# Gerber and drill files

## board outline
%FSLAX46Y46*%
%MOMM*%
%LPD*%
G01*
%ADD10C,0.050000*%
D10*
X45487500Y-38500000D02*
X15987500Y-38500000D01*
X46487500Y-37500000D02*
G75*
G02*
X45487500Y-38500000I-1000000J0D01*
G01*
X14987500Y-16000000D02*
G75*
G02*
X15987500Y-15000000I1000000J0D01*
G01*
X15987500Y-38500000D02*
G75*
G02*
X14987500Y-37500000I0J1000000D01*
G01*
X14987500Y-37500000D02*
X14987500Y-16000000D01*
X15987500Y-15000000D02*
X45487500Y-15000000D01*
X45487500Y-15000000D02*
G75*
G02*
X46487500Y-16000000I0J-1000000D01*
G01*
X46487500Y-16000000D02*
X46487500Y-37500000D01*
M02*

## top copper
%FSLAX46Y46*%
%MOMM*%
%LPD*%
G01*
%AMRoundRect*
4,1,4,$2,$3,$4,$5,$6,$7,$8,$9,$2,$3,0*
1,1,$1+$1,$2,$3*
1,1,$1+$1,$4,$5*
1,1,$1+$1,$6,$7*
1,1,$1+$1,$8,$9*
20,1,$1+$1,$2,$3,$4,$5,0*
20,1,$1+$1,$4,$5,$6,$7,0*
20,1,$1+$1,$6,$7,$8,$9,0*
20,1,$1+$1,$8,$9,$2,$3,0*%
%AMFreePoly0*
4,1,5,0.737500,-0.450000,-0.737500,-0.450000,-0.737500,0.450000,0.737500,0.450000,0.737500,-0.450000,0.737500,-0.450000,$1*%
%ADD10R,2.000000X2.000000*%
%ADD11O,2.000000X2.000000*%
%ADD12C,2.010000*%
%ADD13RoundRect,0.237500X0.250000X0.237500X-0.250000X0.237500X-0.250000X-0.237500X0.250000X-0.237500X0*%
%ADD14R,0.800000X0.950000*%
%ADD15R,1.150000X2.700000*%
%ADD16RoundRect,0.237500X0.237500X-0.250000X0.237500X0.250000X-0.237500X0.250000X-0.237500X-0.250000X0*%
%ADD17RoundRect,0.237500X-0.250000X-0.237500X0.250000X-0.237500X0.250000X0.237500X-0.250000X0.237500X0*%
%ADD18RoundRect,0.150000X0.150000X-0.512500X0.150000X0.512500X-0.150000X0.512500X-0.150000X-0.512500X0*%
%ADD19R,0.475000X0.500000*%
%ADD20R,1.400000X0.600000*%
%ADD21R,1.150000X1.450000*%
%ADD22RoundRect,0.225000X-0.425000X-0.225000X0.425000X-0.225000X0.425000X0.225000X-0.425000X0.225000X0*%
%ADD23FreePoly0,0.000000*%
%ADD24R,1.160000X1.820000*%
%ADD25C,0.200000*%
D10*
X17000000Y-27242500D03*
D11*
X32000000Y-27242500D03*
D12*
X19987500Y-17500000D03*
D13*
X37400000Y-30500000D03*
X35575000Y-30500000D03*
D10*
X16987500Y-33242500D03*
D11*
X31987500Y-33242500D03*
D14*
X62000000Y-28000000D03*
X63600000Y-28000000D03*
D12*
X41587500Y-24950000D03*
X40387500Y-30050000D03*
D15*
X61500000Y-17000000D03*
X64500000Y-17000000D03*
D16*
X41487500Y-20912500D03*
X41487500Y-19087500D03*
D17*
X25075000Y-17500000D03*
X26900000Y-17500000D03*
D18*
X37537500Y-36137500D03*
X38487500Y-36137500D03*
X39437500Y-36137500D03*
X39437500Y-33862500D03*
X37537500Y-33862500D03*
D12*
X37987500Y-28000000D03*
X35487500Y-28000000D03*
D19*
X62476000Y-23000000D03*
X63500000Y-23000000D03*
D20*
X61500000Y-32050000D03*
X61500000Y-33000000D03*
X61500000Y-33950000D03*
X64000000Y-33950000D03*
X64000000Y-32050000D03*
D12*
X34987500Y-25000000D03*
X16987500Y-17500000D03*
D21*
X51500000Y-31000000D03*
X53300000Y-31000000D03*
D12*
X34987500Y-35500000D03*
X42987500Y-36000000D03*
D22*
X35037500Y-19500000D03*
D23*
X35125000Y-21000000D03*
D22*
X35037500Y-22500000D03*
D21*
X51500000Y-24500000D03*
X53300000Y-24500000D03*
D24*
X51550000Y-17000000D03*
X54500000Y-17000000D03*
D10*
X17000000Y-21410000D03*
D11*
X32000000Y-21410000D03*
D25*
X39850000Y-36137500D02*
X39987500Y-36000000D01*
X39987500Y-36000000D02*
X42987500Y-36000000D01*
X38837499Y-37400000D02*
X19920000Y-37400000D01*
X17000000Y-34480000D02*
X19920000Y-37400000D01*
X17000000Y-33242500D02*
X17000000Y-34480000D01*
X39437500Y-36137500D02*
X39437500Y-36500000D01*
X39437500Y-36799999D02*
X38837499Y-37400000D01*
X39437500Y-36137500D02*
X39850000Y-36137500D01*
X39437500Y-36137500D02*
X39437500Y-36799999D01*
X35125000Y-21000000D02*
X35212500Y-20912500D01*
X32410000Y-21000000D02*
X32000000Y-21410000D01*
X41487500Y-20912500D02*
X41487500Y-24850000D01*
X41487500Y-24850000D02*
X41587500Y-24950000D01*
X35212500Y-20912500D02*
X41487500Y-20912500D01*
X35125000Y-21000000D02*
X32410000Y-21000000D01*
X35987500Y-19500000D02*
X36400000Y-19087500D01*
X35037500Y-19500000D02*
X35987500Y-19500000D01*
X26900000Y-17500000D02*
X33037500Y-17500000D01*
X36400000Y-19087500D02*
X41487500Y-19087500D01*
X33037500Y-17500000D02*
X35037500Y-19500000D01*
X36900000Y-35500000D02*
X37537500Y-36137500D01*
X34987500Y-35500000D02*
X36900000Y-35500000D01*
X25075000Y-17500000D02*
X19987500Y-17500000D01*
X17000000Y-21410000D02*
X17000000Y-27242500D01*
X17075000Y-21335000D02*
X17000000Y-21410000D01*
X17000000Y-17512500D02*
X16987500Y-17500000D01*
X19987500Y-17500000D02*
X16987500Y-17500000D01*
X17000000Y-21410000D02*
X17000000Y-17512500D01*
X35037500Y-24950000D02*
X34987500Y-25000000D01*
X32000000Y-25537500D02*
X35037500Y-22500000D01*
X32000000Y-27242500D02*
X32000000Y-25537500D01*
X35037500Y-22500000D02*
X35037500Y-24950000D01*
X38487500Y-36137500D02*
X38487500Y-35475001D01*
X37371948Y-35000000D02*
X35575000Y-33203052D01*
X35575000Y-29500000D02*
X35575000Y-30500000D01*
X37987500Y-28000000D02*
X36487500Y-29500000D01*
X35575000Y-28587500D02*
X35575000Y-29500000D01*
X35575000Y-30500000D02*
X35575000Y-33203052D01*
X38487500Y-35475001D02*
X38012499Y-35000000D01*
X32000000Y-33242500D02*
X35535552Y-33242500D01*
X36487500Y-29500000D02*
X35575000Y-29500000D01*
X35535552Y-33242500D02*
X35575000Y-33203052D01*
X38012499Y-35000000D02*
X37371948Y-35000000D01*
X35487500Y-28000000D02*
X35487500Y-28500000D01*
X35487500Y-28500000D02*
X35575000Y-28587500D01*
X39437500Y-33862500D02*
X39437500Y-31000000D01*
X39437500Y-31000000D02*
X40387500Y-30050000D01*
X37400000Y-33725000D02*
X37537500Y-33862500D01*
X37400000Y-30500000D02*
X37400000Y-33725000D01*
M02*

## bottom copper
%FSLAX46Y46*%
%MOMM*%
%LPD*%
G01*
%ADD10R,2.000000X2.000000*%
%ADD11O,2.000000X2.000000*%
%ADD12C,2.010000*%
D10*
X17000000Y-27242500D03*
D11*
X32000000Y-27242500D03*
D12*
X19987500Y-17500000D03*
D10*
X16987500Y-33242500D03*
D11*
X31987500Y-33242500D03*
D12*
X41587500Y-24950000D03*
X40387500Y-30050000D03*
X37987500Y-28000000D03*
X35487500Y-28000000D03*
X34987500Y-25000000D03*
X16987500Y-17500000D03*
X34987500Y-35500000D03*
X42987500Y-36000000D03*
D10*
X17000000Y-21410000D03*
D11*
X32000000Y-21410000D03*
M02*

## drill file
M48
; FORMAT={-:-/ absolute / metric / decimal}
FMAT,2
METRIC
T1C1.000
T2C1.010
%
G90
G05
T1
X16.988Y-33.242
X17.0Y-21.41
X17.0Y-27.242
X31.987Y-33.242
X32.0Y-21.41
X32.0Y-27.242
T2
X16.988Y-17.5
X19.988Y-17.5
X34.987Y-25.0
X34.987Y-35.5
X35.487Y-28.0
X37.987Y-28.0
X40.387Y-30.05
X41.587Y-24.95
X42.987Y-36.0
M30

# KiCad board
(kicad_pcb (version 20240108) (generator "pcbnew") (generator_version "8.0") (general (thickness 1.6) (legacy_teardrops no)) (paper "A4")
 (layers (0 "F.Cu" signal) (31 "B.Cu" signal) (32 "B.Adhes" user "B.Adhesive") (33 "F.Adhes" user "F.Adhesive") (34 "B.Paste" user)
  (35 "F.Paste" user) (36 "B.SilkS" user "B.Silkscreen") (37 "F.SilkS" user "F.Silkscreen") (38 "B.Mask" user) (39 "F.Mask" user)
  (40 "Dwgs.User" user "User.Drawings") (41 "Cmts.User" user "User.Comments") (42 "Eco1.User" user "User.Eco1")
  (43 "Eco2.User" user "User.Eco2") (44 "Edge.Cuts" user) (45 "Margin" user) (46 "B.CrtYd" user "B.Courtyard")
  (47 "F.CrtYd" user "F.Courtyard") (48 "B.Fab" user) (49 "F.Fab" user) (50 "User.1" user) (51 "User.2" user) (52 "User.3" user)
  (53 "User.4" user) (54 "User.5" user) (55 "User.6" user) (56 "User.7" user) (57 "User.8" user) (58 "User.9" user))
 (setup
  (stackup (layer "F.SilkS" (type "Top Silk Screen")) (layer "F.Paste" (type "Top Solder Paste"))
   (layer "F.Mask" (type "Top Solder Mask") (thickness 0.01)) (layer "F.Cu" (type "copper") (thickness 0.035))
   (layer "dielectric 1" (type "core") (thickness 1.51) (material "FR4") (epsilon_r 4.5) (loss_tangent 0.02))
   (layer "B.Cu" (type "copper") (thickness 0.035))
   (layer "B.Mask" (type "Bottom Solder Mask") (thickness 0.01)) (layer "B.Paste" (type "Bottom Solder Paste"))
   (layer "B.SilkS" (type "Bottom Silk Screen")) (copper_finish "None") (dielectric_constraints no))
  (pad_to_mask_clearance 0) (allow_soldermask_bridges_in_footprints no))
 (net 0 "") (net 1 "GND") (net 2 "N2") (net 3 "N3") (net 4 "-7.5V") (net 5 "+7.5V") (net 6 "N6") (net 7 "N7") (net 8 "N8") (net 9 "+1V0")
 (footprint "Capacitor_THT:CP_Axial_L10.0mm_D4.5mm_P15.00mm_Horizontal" (layer "F.Cu") (at 17 27.2425)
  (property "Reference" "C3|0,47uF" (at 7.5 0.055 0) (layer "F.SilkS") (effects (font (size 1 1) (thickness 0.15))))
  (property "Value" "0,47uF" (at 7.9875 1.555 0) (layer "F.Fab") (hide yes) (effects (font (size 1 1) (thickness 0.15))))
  (pad "2" thru_hole rect (at 0 0) (size 2 2) (drill 1) (layers "*.Cu" "*.Mask") (remove_unused_layers no) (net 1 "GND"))
  (pad "2" thru_hole oval (at 15 0) (size 2 2) (drill 1) (layers "*.Cu" "*.Mask") (remove_unused_layers no) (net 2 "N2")))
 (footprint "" (layer "F.Cu") (at 19.9875 17.5)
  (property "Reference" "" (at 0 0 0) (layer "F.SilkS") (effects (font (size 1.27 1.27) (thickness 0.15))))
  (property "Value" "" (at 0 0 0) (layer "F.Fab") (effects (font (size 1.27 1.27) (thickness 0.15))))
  (pad "4" thru_hole circle (at 0 0 270) (size 2.01 2.01) (drill 1.01) (layers "*.Cu" "*.Mask") (remove_unused_layers no) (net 1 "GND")))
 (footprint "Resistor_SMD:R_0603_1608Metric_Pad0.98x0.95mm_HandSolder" (layer "F.Cu") (at 36.4875 30.5 180)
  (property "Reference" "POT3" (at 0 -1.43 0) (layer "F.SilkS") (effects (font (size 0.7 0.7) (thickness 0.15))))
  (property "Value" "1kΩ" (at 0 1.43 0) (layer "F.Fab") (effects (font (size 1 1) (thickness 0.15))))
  (pad "1" smd roundrect (at -0.9125 0 180) (size 0.975 0.95) (layers "F.Cu" "F.Paste" "F.Mask") (roundrect_rratio 0.25) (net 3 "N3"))
  (pad "2" smd roundrect (at 0.9125 0 180) (size 0.975 0.95) (layers "F.Cu" "F.Paste" "F.Mask") (roundrect_rratio 0.25) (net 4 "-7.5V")))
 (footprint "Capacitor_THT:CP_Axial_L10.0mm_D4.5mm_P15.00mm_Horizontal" (layer "F.Cu") (at 16.9875 33.2425)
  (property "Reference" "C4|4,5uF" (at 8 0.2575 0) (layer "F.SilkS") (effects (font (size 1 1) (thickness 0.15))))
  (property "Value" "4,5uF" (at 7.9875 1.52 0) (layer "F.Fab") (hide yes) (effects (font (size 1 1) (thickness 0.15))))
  (pad "1" thru_hole rect (at 0 0) (size 2 2) (drill 1) (layers "*.Cu" "*.Mask") (remove_unused_layers no) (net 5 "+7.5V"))
  (pad "2" thru_hole oval (at 15 0) (size 2 2) (drill 1) (layers "*.Cu" "*.Mask") (remove_unused_layers no) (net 4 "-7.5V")))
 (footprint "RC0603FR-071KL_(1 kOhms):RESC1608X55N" (layer "F.Cu") (at 62.8 28)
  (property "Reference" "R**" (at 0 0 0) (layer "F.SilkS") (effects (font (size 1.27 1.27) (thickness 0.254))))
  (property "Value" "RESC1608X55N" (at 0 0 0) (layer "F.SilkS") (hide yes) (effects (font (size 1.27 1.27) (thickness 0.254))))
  (pad "1" smd rect (at -0.8 0) (size 0.8 0.95) (layers "F.Cu" "F.Paste" "F.Mask"))
  (pad "2" smd rect (at 0.8 0) (size 0.8 0.95) (layers "F.Cu" "F.Paste" "F.Mask")))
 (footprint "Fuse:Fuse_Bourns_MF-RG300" (layer "F.Cu") (at 41.5875 24.95 -90)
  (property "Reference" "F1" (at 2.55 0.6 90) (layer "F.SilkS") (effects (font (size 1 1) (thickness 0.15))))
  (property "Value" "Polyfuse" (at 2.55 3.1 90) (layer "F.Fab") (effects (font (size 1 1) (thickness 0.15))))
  (pad "1" thru_hole circle (at 0 0 270) (size 2.01 2.01) (drill 1.01) (layers "*.Cu" "*.Mask") (remove_unused_layers no) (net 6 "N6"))
  (pad "2" thru_hole circle (at 5.1 1.2 270) (size 2.01 2.01) (drill 1.01) (layers "*.Cu" "*.Mask") (remove_unused_layers no) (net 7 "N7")))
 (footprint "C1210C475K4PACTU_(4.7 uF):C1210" (layer "F.Cu") (at 63 17)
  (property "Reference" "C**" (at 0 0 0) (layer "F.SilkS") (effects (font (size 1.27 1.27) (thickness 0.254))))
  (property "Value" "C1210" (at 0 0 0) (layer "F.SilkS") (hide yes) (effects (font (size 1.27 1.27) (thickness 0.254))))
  (pad "1" smd rect (at -1.5 0) (size 1.15 2.7) (layers "F.Cu" "F.Paste" "F.Mask"))
  (pad "2" smd rect (at 1.5 0) (size 1.15 2.7) (layers "F.Cu" "F.Paste" "F.Mask")))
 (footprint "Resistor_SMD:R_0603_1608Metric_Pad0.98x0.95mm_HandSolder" (layer "F.Cu") (at 41.4875 20 90)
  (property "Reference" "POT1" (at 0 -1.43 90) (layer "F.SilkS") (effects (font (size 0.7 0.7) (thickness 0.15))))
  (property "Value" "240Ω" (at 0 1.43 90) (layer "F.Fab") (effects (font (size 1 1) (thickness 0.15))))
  (pad "1" smd roundrect (at -0.9125 0 90) (size 0.975 0.95) (layers "F.Cu" "F.Paste" "F.Mask") (roundrect_rratio 0.25) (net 6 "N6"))
  (pad "2" smd roundrect (at 0.9125 0 90) (size 0.975 0.95) (layers "F.Cu" "F.Paste" "F.Mask") (roundrect_rratio 0.25) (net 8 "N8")))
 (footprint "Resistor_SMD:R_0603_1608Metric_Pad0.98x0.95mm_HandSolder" (layer "F.Cu") (at 25.9875 17.5)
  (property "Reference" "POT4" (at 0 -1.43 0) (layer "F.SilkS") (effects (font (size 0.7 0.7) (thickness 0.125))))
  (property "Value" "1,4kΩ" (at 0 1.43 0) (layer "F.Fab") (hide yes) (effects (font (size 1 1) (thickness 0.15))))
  (pad "1" smd roundrect (at -0.9125 0) (size 0.975 0.95) (layers "F.Cu" "F.Paste" "F.Mask") (roundrect_rratio 0.25) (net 1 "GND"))
  (pad "2" smd roundrect (at 0.9125 0) (size 0.975 0.95) (layers "F.Cu" "F.Paste" "F.Mask") (roundrect_rratio 0.25) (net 8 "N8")))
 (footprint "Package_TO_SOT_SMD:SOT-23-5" (layer "F.Cu") (at 38.4875 35 90)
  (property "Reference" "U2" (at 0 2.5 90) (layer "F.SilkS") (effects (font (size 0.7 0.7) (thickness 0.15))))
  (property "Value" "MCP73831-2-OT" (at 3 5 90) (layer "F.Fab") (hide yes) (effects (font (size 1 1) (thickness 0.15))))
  (pad "1" smd roundrect (at -1.1375 -0.95 90) (size 1.325 0.6) (layers "F.Cu" "F.Paste" "F.Mask") (roundrect_rratio 0.25) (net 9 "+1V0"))
  (pad "2" smd roundrect (at -1.1375 0 90) (size 1.325 0.6) (layers "F.Cu" "F.Paste" "F.Mask") (roundrect_rratio 0.25) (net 4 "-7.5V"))
  (pad "3" smd roundrect (at -1.1375 0.95 90) (size 1.325 0.6) (layers "F.Cu" "F.Paste" "F.Mask") (roundrect_rratio 0.25) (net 5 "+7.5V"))
  (pad "4" smd roundrect (at 1.1375 0.95 90) (size 1.325 0.6) (layers "F.Cu" "F.Paste" "F.Mask") (roundrect_rratio 0.25) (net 7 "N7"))
  (pad "5" smd roundrect (at 1.1375 -0.95 90) (size 1.325 0.6) (layers "F.Cu" "F.Paste" "F.Mask") (roundrect_rratio 0.25) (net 3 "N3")))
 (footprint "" (layer "F.Cu") (at 37.9875 28)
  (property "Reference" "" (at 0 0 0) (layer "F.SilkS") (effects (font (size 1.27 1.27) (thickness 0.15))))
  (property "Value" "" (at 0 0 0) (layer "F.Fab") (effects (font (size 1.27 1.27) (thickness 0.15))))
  (pad "1" thru_hole circle (at 0 0 270) (size 2.01 2.01) (drill 1.01) (layers "*.Cu" "*.Mask") (remove_unused_layers no) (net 4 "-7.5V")))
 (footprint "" (layer "F.Cu") (at 35.4875 28)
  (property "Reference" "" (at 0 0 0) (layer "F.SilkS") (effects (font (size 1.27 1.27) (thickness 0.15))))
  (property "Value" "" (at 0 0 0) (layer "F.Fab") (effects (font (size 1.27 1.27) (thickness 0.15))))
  (pad "1" thru_hole circle (at 0 0 270) (size 2.01 2.01) (drill 1.01) (layers "*.Cu" "*.Mask") (remove_unused_layers no) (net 4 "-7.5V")))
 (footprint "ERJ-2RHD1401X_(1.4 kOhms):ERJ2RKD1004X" (layer "F.Cu") (at 62.988 23)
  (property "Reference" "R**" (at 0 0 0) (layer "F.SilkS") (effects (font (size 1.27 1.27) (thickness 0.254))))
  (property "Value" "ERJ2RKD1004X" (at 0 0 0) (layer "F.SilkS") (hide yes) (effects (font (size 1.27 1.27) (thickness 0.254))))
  (pad "1" smd rect (at -0.512 0) (size 0.475 0.5) (layers "F.Cu" "F.Paste" "F.Mask"))
  (pad "2" smd rect (at 0.512 0) (size 0.475 0.5) (layers "F.Cu" "F.Paste" "F.Mask")))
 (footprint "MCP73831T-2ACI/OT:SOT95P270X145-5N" (layer "F.Cu") (at 62.75 33)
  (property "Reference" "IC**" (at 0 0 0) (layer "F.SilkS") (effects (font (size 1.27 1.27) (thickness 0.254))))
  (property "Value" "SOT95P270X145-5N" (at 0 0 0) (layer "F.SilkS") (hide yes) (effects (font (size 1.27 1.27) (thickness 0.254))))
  (pad "1" smd rect (at -1.25 -0.95 90) (size 0.6 1.4) (layers "F.Cu" "F.Paste" "F.Mask"))
  (pad "2" smd rect (at -1.25 0 90) (size 0.6 1.4) (layers "F.Cu" "F.Paste" "F.Mask"))
  (pad "3" smd rect (at -1.25 0.95 90) (size 0.6 1.4) (layers "F.Cu" "F.Paste" "F.Mask"))
  (pad "4" smd rect (at 1.25 0.95 90) (size 0.6 1.4) (layers "F.Cu" "F.Paste" "F.Mask"))
  (pad "5" smd rect (at 1.25 -0.95 90) (size 0.6 1.4) (layers "F.Cu" "F.Paste" "F.Mask")))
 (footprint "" (layer "F.Cu") (at 34.9875 25)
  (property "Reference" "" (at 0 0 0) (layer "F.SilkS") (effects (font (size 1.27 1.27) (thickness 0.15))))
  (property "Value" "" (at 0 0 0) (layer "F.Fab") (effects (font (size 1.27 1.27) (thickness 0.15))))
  (pad "1" thru_hole circle (at 0 0 270) (size 2.01 2.01) (drill 1.01) (layers "*.Cu" "*.Mask") (remove_unused_layers no) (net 2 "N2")))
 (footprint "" (layer "F.Cu") (at 16.9875 17.5)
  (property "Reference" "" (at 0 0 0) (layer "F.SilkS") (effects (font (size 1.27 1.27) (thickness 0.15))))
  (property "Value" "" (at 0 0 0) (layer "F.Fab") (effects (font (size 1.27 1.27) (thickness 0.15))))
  (pad "3" thru_hole circle (at 0 0 270) (size 2.01 2.01) (drill 1.01) (layers "*.Cu" "*.Mask") (remove_unused_layers no) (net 1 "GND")))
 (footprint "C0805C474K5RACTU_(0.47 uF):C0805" (layer "F.Cu") (at 52.4 31)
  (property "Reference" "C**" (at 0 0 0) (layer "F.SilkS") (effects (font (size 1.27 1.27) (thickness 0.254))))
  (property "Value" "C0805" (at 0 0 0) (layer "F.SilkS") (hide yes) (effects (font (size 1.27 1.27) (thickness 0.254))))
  (pad "1" smd rect (at -0.9 0) (size 1.15 1.45) (layers "F.Cu" "F.Paste" "F.Mask"))
  (pad "2" smd rect (at 0.9 0) (size 1.15 1.45) (layers "F.Cu" "F.Paste" "F.Mask")))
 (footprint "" (layer "F.Cu") (at 34.9875 35.5)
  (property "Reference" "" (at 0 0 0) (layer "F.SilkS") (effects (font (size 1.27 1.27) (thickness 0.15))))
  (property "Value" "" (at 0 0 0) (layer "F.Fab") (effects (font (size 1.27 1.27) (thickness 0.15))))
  (pad "1" thru_hole circle (at 0 0 270) (size 2.01 2.01) (drill 1.01) (layers "*.Cu" "*.Mask") (remove_unused_layers no) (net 9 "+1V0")))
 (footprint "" (layer "F.Cu") (at 42.9875 36)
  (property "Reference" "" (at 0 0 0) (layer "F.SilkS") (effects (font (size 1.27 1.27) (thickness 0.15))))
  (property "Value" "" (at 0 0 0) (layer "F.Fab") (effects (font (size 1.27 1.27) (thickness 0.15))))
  (pad "2" thru_hole circle (at 0 0 270) (size 2.01 2.01) (drill 1.01) (layers "*.Cu" "*.Mask") (remove_unused_layers no) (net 5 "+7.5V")))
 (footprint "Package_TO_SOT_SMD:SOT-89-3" (layer "F.Cu") (at 36.9875 21)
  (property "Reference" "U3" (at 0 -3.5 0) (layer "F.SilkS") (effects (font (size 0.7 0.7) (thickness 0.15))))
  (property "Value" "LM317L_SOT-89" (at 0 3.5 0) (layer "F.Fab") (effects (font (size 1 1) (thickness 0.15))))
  (pad "1" smd roundrect (at -1.95 -1.5) (size 1.3 0.9) (layers "F.Cu" "F.Paste" "F.Mask") (roundrect_rratio 0.25) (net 8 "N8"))
  (pad "2" smd custom (at -1.8625 0) (size 1.475 0.9) (layers "F.Cu" "F.Paste" "F.Mask") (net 6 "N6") (zone_connect 2)
   (thermal_bridge_angle 45) (options (clearance outline) (anchor rect)) (primitives))
  (pad "3" smd roundrect (at -1.95 1.5) (size 1.3 0.9) (layers "F.Cu" "F.Paste" "F.Mask") (roundrect_rratio 0.25) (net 2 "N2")))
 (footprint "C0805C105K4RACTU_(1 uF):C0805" (layer "F.Cu") (at 52.4 24.5)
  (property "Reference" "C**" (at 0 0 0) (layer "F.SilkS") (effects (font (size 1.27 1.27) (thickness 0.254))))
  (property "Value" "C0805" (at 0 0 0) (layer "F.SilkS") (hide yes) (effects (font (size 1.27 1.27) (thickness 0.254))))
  (pad "1" smd rect (at -0.9 0) (size 1.15 1.45) (layers "F.Cu" "F.Paste" "F.Mask"))
  (pad "2" smd rect (at 0.9 0) (size 1.15 1.45) (layers "F.Cu" "F.Paste" "F.Mask")))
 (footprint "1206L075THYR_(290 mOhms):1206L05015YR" (layer "F.Cu") (at 53.025 17)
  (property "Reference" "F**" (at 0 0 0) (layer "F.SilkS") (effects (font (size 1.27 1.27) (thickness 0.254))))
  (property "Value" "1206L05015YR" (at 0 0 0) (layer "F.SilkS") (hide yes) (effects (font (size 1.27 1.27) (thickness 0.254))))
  (pad "1" smd rect (at -1.475 0) (size 1.16 1.82) (layers "F.Cu" "F.Paste" "F.Mask"))
  (pad "2" smd rect (at 1.475 0) (size 1.16 1.82) (layers "F.Cu" "F.Paste" "F.Mask")))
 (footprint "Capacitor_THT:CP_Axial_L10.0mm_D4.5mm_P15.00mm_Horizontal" (layer "F.Cu") (at 17 21.41)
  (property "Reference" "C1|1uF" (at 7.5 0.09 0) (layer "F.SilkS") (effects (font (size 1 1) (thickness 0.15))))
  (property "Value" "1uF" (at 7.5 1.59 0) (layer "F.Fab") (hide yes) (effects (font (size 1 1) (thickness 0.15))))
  (pad "1" thru_hole rect (at 0 0) (size 2 2) (drill 1) (layers "*.Cu" "*.Mask") (remove_unused_layers no) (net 1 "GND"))
  (pad "2" thru_hole oval (at 15 0) (size 2 2) (drill 1) (layers "*.Cu" "*.Mask") (remove_unused_layers no) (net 6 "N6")))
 (gr_line (start 45.4875 38.5) (end 15.9875 38.5) (stroke (width 0.05) (type default)) (layer "Edge.Cuts"))
 (gr_arc (start 46.4875 37.5) (mid 46.194607 38.207107) (end 45.4875 38.5) (stroke (width 0.05) (type default)) (layer "Edge.Cuts"))
 (gr_arc (start 14.9875 16) (mid 15.280393 15.292893) (end 15.9875 15) (stroke (width 0.05) (type default)) (layer "Edge.Cuts"))
 (gr_arc (start 15.9875 38.5) (mid 15.280393 38.207107) (end 14.9875 37.5) (stroke (width 0.05) (type default)) (layer "Edge.Cuts"))
 (gr_line (start 14.9875 37.5) (end 14.9875 16) (stroke (width 0.05) (type default)) (layer "Edge.Cuts"))
 (gr_line (start 15.9875 15) (end 45.4875 15) (stroke (width 0.05) (type default)) (layer "Edge.Cuts"))
 (gr_arc (start 45.4875 15) (mid 46.194607 15.292893) (end 46.4875 16) (stroke (width 0.05) (type default)) (layer "Edge.Cuts"))
 (gr_line (start 46.4875 16) (end 46.4875 37.5) (stroke (width 0.05) (type default)) (layer "Edge.Cuts"))
 (segment (start 39.85 36.1375) (end 39.9875 36) (width 0.2) (layer "F.Cu") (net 5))
 (segment (start 39.9875 36) (end 42.9875 36) (width 0.2) (layer "F.Cu") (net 5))
 (segment (start 38.837499 37.4) (end 19.92 37.4) (width 0.2) (layer "F.Cu") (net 5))
 (segment (start 17 34.48) (end 19.92 37.4) (width 0.2) (layer "F.Cu") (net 5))
 (segment (start 17 33.2425) (end 17 34.48) (width 0.2) (layer "F.Cu") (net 5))
 (segment (start 39.4375 36.1375) (end 39.4375 36.5) (width 0.2) (layer "F.Cu") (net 5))
 (segment (start 39.4375 36.799999) (end 38.837499 37.4) (width 0.2) (layer "F.Cu") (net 5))
 (segment (start 39.4375 36.1375) (end 39.85 36.1375) (width 0.2) (layer "F.Cu") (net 5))
 (segment (start 39.4375 36.1375) (end 39.4375 36.799999) (width 0.2) (layer "F.Cu") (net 5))
 (segment (start 35.125 21) (end 35.2125 20.9125) (width 0.2) (layer "F.Cu") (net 6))
 (segment (start 32.41 21) (end 32 21.41) (width 0.2) (layer "F.Cu") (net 6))
 (segment (start 41.4875 20.9125) (end 41.4875 24.85) (width 0.2) (layer "F.Cu") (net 6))
 (segment (start 41.4875 24.85) (end 41.5875 24.95) (width 0.2) (layer "F.Cu") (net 6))
 (segment (start 35.2125 20.9125) (end 41.4875 20.9125) (width 0.2) (layer "F.Cu") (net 6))
 (segment (start 35.125 21) (end 32.41 21) (width 0.2) (layer "F.Cu") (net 6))
 (segment (start 35.9875 19.5) (end 36.4 19.0875) (width 0.2) (layer "F.Cu") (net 8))
 (segment (start 35.0375 19.5) (end 35.9875 19.5) (width 0.2) (layer "F.Cu") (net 8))
 (segment (start 26.9 17.5) (end 33.0375 17.5) (width 0.2) (layer "F.Cu") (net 8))
 (segment (start 36.4 19.0875) (end 41.4875 19.0875) (width 0.2) (layer "F.Cu") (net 8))
 (segment (start 33.0375 17.5) (end 35.0375 19.5) (width 0.2) (layer "F.Cu") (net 8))
 (segment (start 36.9 35.5) (end 37.5375 36.1375) (width 0.2) (layer "F.Cu") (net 9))
 (segment (start 34.9875 35.5) (end 36.9 35.5) (width 0.2) (layer "F.Cu") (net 9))
 (segment (start 25.075 17.5) (end 19.9875 17.5) (width 0.2) (layer "F.Cu") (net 1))
 (segment (start 17 21.41) (end 17 27.2425) (width 0.2) (layer "F.Cu") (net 1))
 (segment (start 17.075 21.335) (end 17 21.41) (width 0.2) (layer "F.Cu") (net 1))
 (segment (start 17 17.5125) (end 16.9875 17.5) (width 0.2) (layer "F.Cu") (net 1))
 (segment (start 19.9875 17.5) (end 16.9875 17.5) (width 0.2) (layer "F.Cu") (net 1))
 (segment (start 17 21.41) (end 17 17.5125) (width 0.2) (layer "F.Cu") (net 1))
 (segment (start 35.0375 24.95) (end 34.9875 25) (width 0.2) (layer "F.Cu") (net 2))
 (segment (start 32 25.5375) (end 35.0375 22.5) (width 0.2) (layer "F.Cu") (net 2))
 (segment (start 32 27.2425) (end 32 25.5375) (width 0.2) (layer "F.Cu") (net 2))
 (segment (start 35.0375 22.5) (end 35.0375 24.95) (width 0.2) (layer "F.Cu") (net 2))
 (segment (start 38.4875 36.1375) (end 38.4875 35.475001) (width 0.2) (layer "F.Cu") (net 4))
 (segment (start 37.371948 35) (end 35.575 33.203052) (width 0.2) (layer "F.Cu") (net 4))
 (segment (start 35.575 29.5) (end 35.575 30.5) (width 0.2) (layer "F.Cu") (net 4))
 (segment (start 37.9875 28) (end 36.4875 29.5) (width 0.2) (layer "F.Cu") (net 4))
 (segment (start 35.575 28.5875) (end 35.575 29.5) (width 0.2) (layer "F.Cu") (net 4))
 (segment (start 35.575 30.5) (end 35.575 33.203052) (width 0.2) (layer "F.Cu") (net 4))
 (segment (start 38.4875 35.475001) (end 38.012499 35) (width 0.2) (layer "F.Cu") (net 4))
 (segment (start 32 33.2425) (end 35.535552 33.2425) (width 0.2) (layer "F.Cu") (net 4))
 (segment (start 36.4875 29.5) (end 35.575 29.5) (width 0.2) (layer "F.Cu") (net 4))
 (segment (start 35.535552 33.2425) (end 35.575 33.203052) (width 0.2) (layer "F.Cu") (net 4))
 (segment (start 38.012499 35) (end 37.371948 35) (width 0.2) (layer "F.Cu") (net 4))
 (segment (start 35.4875 28) (end 35.4875 28.5) (width 0.2) (layer "F.Cu") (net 4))
 (segment (start 35.4875 28.5) (end 35.575 28.5875) (width 0.2) (layer "F.Cu") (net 4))
 (segment (start 39.4375 33.8625) (end 39.4375 31) (width 0.2) (layer "F.Cu") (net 7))
 (segment (start 39.4375 31) (end 40.3875 30.05) (width 0.2) (layer "F.Cu") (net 7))
 (segment (start 37.4 33.725) (end 37.5375 33.8625) (width 0.2) (layer "F.Cu") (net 3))
 (segment (start 37.4 30.5) (end 37.4 33.725) (width 0.2) (layer "F.Cu") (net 3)))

